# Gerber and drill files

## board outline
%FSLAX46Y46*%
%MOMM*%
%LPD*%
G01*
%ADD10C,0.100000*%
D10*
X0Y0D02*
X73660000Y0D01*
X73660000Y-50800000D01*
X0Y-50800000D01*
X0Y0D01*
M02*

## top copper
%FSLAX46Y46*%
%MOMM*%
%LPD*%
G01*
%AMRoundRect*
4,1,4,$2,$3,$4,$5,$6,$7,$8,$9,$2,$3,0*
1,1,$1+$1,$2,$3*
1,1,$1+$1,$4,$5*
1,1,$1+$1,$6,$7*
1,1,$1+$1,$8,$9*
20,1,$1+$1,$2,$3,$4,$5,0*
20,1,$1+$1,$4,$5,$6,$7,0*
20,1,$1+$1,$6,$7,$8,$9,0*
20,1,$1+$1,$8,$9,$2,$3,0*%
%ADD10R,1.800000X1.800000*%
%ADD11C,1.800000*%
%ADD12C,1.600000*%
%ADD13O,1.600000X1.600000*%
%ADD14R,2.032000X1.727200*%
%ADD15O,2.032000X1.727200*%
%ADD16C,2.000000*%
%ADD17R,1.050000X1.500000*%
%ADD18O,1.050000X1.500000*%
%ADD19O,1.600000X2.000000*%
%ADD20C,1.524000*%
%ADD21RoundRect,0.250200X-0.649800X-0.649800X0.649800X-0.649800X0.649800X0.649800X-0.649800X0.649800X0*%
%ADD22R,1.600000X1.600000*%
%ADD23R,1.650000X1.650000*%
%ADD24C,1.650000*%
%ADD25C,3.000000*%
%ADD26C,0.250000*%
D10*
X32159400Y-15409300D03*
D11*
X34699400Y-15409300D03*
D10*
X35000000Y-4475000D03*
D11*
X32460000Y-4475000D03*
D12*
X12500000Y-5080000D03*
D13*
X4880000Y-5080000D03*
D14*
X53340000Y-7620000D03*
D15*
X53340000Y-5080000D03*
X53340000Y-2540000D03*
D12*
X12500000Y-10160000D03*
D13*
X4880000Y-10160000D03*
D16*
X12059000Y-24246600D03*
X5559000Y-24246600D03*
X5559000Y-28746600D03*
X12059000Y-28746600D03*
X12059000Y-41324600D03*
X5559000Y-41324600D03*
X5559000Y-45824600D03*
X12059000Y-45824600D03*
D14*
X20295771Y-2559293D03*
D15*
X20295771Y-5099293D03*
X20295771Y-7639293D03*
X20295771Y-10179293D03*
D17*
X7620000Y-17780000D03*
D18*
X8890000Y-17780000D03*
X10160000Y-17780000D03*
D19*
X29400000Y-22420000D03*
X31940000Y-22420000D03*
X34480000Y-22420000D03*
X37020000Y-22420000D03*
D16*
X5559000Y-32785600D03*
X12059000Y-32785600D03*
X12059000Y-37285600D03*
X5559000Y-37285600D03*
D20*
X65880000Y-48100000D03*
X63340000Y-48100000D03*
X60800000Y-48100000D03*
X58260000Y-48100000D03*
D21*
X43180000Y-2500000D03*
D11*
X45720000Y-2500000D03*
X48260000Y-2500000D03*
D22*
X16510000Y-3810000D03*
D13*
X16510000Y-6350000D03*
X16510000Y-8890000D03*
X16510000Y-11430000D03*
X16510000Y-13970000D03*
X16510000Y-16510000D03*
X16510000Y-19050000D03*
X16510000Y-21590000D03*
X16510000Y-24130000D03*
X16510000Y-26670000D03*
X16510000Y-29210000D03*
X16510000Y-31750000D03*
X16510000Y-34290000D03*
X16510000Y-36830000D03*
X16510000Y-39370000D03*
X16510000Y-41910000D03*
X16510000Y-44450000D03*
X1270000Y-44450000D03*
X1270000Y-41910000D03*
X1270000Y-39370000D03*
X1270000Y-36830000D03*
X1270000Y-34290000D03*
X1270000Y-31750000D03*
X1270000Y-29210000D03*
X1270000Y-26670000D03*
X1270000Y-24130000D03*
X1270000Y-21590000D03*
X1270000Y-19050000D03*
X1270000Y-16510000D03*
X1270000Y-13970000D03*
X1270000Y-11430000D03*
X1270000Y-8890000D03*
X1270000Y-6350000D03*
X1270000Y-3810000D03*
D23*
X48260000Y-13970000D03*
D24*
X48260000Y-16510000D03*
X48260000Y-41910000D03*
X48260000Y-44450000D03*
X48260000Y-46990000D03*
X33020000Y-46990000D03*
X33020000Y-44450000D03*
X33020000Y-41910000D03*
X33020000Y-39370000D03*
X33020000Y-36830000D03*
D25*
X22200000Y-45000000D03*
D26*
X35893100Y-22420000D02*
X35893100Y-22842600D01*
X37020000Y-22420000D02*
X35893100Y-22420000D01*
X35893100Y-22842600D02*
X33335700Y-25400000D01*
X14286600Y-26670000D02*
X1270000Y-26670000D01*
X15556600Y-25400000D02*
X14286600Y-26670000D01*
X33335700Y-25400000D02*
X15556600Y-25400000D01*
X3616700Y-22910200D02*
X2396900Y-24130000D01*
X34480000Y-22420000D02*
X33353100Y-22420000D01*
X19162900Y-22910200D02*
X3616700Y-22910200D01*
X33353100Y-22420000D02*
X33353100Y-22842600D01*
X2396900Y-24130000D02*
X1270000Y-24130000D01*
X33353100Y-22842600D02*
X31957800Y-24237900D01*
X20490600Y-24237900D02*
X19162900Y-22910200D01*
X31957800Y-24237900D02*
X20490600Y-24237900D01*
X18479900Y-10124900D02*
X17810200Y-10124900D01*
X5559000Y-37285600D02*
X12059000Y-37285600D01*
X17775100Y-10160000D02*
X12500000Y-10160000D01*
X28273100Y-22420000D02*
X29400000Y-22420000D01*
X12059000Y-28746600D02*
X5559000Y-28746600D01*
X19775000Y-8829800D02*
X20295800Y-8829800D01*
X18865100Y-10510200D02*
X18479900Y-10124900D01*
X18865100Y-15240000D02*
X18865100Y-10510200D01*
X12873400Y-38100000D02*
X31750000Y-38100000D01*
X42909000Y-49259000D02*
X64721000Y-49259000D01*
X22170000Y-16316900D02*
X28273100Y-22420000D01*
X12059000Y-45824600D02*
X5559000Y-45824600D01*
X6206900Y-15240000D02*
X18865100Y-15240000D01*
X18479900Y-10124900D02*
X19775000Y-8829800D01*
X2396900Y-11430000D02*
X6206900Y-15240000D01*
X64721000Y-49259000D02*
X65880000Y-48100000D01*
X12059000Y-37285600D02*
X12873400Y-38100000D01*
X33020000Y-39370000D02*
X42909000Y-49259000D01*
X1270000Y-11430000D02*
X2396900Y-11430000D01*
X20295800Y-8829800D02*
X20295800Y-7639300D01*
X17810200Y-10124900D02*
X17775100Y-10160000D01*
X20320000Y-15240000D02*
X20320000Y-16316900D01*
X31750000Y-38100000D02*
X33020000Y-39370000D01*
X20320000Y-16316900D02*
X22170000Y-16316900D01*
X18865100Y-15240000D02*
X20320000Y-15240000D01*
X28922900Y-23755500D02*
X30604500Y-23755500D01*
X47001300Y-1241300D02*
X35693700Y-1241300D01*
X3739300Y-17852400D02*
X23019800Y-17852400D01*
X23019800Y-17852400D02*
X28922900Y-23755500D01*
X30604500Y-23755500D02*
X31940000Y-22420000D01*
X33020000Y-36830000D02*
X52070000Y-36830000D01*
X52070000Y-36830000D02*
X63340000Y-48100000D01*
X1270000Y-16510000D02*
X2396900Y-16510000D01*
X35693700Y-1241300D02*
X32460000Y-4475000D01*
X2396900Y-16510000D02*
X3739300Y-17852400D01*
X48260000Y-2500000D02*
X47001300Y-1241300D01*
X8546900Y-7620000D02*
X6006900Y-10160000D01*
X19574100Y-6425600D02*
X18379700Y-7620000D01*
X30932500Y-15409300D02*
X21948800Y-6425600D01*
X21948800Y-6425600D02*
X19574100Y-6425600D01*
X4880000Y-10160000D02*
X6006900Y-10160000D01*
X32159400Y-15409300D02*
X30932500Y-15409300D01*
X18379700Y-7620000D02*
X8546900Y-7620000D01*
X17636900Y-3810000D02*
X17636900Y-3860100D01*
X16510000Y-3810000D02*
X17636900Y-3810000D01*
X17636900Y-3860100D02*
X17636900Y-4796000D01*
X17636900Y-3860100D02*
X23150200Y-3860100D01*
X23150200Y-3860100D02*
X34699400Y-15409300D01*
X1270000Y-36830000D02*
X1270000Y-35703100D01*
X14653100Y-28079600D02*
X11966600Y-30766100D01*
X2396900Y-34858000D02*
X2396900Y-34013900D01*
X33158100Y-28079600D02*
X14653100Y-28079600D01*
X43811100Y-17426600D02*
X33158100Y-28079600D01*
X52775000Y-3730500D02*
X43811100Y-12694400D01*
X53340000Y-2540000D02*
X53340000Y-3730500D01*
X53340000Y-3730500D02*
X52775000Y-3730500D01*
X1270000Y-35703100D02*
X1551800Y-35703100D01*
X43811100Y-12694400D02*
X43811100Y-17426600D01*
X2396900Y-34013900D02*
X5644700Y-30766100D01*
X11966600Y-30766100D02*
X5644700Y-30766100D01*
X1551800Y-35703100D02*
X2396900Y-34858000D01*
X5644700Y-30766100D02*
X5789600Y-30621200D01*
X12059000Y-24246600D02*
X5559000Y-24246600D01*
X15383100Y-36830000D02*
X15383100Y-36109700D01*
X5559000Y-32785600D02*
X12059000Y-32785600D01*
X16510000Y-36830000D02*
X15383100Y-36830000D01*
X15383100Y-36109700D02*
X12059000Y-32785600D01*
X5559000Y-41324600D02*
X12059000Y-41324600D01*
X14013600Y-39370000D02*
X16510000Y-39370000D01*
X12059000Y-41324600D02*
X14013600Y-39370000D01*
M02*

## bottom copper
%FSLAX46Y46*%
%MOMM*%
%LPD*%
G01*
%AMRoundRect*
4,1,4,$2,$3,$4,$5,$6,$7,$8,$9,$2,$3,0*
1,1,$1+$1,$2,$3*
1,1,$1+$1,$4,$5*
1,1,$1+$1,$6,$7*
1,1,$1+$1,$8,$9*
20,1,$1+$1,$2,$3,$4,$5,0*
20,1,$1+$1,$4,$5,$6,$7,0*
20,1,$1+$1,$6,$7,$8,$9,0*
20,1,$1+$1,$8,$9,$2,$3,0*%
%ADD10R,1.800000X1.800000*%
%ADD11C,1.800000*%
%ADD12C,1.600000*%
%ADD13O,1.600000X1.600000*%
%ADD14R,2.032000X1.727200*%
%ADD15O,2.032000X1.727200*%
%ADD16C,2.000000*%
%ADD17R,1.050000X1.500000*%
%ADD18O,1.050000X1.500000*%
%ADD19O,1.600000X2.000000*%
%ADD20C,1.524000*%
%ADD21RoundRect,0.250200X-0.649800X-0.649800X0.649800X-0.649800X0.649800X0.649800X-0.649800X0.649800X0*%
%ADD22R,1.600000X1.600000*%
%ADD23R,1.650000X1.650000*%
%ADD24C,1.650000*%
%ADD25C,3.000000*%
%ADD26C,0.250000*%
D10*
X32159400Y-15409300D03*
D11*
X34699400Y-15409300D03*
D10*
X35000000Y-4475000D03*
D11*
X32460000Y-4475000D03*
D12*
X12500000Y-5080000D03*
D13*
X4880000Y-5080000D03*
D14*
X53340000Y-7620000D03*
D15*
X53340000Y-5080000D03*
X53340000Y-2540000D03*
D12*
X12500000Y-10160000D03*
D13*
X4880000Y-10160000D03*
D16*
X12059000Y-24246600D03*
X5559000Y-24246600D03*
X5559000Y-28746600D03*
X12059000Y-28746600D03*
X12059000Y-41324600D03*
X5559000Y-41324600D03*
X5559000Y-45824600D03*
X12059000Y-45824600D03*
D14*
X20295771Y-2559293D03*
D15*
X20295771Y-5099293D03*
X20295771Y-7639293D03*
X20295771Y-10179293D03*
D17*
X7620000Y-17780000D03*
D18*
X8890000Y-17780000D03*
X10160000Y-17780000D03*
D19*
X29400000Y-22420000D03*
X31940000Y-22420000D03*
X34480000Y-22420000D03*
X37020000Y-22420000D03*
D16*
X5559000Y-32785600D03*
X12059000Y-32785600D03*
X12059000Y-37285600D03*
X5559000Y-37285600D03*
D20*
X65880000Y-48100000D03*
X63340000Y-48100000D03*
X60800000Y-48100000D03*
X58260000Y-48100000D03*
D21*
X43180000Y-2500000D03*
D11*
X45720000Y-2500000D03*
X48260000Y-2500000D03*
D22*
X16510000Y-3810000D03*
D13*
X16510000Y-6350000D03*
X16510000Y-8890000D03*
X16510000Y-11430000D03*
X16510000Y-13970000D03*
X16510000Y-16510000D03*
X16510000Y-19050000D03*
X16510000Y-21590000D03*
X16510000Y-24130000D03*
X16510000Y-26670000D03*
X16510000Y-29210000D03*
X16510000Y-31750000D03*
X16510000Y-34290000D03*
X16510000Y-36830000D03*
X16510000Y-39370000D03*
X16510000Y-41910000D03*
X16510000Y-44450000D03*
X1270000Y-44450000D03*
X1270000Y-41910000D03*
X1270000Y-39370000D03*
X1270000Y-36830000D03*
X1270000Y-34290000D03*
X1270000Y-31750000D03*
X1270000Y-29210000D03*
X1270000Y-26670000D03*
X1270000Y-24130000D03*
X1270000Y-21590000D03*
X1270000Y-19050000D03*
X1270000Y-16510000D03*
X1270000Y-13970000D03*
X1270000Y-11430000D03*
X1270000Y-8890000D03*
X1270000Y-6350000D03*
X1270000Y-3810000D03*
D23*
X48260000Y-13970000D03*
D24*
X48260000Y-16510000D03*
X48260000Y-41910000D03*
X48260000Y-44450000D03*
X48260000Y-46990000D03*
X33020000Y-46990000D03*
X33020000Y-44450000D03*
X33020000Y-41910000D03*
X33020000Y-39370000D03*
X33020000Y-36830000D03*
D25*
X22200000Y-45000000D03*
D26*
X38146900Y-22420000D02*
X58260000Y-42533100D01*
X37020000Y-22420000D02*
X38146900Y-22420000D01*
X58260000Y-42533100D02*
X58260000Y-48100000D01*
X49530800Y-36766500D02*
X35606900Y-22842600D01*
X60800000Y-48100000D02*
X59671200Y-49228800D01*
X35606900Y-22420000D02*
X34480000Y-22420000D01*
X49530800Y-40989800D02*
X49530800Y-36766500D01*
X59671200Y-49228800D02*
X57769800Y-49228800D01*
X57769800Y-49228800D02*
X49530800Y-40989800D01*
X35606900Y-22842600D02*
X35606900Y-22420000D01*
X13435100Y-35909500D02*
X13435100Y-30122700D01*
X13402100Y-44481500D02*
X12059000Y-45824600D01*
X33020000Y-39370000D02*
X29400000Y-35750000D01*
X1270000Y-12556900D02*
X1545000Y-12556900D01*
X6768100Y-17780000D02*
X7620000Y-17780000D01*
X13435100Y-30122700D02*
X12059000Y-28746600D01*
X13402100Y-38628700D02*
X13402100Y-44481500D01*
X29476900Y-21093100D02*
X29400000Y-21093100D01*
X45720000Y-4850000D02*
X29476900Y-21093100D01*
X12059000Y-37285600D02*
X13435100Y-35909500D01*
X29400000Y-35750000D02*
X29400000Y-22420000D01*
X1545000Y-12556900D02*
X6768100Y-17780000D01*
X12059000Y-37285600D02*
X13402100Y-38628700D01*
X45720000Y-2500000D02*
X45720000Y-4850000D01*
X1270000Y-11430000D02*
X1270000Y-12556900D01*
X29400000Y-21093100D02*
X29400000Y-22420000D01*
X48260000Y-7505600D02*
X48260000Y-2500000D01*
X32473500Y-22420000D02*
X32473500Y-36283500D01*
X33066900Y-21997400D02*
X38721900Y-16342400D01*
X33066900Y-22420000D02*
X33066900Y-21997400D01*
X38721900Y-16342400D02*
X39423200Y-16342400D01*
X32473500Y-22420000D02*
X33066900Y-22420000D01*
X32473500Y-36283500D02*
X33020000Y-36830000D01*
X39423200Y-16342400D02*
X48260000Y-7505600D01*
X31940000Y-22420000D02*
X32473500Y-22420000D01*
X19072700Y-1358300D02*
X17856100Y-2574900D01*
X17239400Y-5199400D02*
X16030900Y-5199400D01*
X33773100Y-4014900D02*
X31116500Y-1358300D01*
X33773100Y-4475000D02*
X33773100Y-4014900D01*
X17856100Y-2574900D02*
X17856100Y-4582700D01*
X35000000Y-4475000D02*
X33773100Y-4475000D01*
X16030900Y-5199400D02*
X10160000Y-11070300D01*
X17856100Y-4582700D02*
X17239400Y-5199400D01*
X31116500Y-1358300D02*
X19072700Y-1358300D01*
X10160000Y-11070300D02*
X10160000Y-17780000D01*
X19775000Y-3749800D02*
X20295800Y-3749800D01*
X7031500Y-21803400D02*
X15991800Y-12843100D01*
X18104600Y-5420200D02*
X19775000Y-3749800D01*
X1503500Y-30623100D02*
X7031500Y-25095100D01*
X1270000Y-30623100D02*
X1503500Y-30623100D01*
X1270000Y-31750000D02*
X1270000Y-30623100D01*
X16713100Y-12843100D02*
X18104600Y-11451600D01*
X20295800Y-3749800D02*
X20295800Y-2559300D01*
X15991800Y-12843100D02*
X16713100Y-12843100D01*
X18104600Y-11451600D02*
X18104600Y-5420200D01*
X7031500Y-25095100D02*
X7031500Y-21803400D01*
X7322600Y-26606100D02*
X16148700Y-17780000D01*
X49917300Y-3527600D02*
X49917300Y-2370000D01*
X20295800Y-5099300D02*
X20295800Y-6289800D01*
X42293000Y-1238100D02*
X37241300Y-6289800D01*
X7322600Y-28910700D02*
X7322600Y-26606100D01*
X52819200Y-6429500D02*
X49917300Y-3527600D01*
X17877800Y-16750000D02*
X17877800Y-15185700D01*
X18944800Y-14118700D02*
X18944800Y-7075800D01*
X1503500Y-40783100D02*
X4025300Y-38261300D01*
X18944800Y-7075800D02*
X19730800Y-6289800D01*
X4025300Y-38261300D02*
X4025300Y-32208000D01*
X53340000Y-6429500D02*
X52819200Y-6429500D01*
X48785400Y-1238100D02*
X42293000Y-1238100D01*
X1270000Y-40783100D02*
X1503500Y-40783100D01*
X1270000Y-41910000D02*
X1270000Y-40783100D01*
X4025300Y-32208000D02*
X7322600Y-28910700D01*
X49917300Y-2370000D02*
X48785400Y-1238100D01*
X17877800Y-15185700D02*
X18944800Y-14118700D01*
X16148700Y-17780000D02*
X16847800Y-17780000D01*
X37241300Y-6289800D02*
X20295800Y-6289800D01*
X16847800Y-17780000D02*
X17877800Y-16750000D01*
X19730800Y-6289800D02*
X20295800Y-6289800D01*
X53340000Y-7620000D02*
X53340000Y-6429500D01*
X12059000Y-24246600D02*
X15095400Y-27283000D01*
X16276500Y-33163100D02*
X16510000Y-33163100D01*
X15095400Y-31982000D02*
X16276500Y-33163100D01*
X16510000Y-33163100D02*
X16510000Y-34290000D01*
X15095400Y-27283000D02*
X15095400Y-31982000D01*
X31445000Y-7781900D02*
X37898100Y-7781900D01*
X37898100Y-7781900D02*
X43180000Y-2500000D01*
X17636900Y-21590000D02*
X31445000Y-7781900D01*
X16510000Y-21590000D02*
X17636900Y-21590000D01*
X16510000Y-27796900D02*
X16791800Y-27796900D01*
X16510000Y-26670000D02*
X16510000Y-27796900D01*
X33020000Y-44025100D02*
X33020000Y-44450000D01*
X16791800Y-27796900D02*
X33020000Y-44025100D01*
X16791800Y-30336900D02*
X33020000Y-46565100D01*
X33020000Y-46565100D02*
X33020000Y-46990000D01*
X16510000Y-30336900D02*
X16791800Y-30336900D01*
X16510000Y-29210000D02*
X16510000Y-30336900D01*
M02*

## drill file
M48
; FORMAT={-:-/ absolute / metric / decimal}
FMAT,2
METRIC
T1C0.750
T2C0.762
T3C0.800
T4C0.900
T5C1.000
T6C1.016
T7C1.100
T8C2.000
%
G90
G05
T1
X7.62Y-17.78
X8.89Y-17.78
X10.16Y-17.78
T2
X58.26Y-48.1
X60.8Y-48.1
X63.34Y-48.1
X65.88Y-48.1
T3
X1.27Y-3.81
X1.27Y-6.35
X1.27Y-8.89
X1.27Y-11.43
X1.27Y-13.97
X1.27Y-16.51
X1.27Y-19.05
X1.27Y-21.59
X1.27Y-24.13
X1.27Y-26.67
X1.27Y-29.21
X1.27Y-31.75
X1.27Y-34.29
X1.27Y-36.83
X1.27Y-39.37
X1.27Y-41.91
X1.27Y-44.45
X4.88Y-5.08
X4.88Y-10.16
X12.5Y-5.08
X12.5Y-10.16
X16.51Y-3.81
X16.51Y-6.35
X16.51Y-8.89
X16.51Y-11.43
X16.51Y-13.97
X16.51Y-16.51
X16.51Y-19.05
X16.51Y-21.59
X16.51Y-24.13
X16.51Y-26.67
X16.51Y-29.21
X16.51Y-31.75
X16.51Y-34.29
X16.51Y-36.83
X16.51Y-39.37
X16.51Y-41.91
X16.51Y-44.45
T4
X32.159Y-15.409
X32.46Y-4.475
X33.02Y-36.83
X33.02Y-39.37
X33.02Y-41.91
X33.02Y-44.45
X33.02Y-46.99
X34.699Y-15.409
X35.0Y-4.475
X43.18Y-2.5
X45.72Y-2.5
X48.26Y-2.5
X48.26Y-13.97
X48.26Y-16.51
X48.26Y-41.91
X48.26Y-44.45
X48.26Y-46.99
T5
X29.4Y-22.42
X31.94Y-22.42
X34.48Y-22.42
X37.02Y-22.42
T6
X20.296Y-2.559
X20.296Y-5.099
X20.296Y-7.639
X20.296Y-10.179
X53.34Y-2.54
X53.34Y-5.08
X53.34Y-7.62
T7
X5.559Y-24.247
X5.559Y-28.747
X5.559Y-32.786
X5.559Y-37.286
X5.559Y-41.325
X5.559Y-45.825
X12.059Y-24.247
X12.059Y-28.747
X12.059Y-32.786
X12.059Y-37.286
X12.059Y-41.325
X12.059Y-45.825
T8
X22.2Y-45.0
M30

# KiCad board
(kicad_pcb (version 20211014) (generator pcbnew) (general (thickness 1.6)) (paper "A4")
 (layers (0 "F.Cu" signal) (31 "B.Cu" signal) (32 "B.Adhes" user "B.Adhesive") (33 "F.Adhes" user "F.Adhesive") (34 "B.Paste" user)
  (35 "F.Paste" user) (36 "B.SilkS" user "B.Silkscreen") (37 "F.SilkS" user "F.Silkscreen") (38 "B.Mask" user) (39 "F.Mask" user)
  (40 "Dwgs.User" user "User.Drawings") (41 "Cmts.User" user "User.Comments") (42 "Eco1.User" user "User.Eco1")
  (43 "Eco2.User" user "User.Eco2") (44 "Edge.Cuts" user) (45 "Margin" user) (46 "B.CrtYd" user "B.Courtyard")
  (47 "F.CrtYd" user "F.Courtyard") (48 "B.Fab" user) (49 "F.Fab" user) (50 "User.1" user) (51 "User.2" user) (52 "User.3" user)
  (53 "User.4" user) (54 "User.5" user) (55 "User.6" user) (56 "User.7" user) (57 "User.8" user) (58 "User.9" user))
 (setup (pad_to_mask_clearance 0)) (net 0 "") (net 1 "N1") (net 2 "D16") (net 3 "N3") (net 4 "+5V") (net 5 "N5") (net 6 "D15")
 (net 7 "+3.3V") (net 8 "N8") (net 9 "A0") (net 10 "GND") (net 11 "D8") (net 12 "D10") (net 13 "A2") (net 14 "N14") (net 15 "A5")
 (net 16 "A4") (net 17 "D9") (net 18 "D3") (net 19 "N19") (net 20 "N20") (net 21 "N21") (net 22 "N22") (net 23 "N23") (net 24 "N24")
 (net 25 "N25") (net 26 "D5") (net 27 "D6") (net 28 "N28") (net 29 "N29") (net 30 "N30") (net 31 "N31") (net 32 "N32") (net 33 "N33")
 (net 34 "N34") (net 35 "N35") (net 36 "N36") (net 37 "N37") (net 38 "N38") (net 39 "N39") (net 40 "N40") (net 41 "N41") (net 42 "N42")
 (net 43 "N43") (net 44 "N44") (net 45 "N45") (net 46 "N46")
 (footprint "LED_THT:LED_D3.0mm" (layer "F.Cu") (at 32.1594 15.4093)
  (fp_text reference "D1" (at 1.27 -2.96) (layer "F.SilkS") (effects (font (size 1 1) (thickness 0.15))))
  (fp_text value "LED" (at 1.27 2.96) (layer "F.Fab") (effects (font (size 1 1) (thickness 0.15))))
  (pad "1" thru_hole rect (at 0 0) (size 1.8 1.8) (drill 0.9) (layers *.Cu *.Mask) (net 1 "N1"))
  (pad "2" thru_hole circle (at 2.54 0) (size 1.8 1.8) (drill 0.9) (layers *.Cu *.Mask) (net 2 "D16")))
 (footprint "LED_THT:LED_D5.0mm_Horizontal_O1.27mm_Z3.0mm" (layer "F.Cu") (at 35 4.475 180)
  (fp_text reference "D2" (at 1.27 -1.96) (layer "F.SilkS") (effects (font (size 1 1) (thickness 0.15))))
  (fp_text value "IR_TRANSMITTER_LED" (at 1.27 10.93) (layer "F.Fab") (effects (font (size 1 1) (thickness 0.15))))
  (pad "1" thru_hole rect (at 0 0 180) (size 1.8 1.8) (drill 0.9) (layers *.Cu *.Mask) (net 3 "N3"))
  (pad "2" thru_hole circle (at 2.54 0 180) (size 1.8 1.8) (drill 0.9) (layers *.Cu *.Mask) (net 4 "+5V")))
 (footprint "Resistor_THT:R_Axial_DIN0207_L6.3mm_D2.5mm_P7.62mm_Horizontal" (layer "F.Cu") (at 12.5 5.08 180)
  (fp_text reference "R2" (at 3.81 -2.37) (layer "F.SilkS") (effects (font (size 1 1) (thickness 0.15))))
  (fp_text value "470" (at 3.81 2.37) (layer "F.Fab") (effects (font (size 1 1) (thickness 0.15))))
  (pad "1" thru_hole circle (at 0 0 180) (size 1.6 1.6) (drill 0.8) (layers *.Cu *.Mask) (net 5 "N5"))
  (pad "2" thru_hole oval (at 7.62 0 180) (size 1.6 1.6) (drill 0.8) (layers *.Cu *.Mask) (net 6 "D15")))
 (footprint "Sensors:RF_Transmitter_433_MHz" (layer "F.Cu") (at 53.34 5.08 90)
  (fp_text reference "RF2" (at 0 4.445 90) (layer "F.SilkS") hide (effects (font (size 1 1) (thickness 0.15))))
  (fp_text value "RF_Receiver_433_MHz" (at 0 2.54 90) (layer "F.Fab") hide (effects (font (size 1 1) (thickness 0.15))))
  (pad "1" thru_hole rect locked (at -2.54 0 180) (size 2.032 1.7272) (drill 1.016) (layers *.Cu *.Mask "F.SilkS") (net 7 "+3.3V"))
  (pad "2" thru_hole oval locked (at 0 0 180) (size 2.032 1.7272) (drill 1.016) (layers *.Cu *.Mask "F.SilkS") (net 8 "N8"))
  (pad "3" thru_hole oval locked (at 2.54 0 180) (size 2.032 1.7272) (drill 1.016) (layers *.Cu *.Mask "F.SilkS") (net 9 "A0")))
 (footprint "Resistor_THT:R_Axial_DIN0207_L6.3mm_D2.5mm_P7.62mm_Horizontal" (layer "F.Cu") (at 12.5 10.16 180)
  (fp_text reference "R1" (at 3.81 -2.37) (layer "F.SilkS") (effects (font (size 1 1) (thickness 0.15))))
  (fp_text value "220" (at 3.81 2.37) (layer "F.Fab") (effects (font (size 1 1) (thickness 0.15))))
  (pad "1" thru_hole circle (at 0 0 180) (size 1.6 1.6) (drill 0.8) (layers *.Cu *.Mask) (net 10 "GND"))
  (pad "2" thru_hole oval (at 7.62 0 180) (size 1.6 1.6) (drill 0.8) (layers *.Cu *.Mask) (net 1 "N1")))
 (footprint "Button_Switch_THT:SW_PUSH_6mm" (layer "F.Cu") (at 5.559 24.2466)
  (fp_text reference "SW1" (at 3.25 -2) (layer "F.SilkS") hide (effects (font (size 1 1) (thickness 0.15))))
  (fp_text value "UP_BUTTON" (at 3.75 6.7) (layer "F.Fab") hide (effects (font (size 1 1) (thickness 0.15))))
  (pad "1" thru_hole circle (at 6.5 0 90) (size 2 2) (drill 1.1) (layers *.Cu *.Mask) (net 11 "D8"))
  (pad "1" thru_hole circle (at 0 0 90) (size 2 2) (drill 1.1) (layers *.Cu *.Mask) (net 11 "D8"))
  (pad "2" thru_hole circle (at 0 4.5 90) (size 2 2) (drill 1.1) (layers *.Cu *.Mask) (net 10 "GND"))
  (pad "2" thru_hole circle (at 6.5 4.5 90) (size 2 2) (drill 1.1) (layers *.Cu *.Mask) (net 10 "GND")))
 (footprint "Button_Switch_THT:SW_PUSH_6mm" (layer "F.Cu") (at 5.559 41.3246)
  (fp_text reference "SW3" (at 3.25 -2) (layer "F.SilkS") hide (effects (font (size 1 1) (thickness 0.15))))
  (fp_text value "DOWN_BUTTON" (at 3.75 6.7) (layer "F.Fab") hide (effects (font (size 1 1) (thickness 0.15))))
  (pad "1" thru_hole circle (at 6.5 0 90) (size 2 2) (drill 1.1) (layers *.Cu *.Mask) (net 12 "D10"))
  (pad "1" thru_hole circle (at 0 0 90) (size 2 2) (drill 1.1) (layers *.Cu *.Mask) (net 12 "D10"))
  (pad "2" thru_hole circle (at 0 4.5 90) (size 2 2) (drill 1.1) (layers *.Cu *.Mask) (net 10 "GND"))
  (pad "2" thru_hole circle (at 6.5 4.5 90) (size 2 2) (drill 1.1) (layers *.Cu *.Mask) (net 10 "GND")))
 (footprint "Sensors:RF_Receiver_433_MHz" (layer "F.Cu") (at 20.32 7.62 -90)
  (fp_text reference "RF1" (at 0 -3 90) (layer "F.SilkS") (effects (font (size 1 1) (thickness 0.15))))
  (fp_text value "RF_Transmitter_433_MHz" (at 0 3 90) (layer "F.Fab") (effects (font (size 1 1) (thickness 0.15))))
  (pad "1" thru_hole rect locked (at -5.060707 0.024229) (size 2.032 1.7272) (drill 1.016) (layers *.Cu *.Mask "F.SilkS") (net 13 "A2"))
  (pad "2" thru_hole oval locked (at -2.520707 0.024229) (size 2.032 1.7272) (drill 1.016) (layers *.Cu *.Mask "F.SilkS") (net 7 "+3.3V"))
  (pad "3" thru_hole oval locked (at 0.019293 0.024229) (size 2.032 1.7272) (drill 1.016) (layers *.Cu *.Mask "F.SilkS") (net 10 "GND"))
  (pad "4" thru_hole oval locked (at 2.559293 0.024229) (size 2.032 1.7272) (drill 1.016) (layers *.Cu *.Mask "F.SilkS")))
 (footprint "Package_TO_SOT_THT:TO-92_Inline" (layer "F.Cu") (at 7.62 17.78)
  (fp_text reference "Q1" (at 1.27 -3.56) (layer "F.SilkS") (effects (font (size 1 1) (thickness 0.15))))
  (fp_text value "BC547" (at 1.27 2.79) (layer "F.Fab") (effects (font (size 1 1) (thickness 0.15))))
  (pad "1" thru_hole rect (at 0 0) (size 1.05 1.5) (drill 0.75) (layers *.Cu *.Mask) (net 10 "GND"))
  (pad "2" thru_hole oval (at 1.27 0) (size 1.05 1.5) (drill 0.75) (layers *.Cu *.Mask) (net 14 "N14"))
  (pad "3" thru_hole oval (at 2.54 0) (size 1.05 1.5) (drill 0.75) (layers *.Cu *.Mask) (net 3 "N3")))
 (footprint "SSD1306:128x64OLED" (layer "F.Cu") (at 33.02 33.02)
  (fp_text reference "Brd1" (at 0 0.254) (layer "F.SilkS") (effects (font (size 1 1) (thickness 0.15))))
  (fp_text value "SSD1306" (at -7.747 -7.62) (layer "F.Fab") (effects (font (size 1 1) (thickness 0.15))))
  (pad "1" thru_hole oval locked (at -3.62 -10.6 90) (size 2 1.6) (drill 1) (layers *.Cu *.Mask) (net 10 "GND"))
  (pad "2" thru_hole oval locked (at -1.08 -10.6 90) (size 2 1.6) (drill 1) (layers *.Cu *.Mask) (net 4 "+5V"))
  (pad "3" thru_hole oval locked (at 1.46 -10.6 90) (size 2 1.6) (drill 1) (layers *.Cu *.Mask) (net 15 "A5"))
  (pad "4" thru_hole oval locked (at 4 -10.6 90) (size 2 1.6) (drill 1) (layers *.Cu *.Mask) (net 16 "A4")))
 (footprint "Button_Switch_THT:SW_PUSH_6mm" (layer "F.Cu") (at 5.559 32.7856)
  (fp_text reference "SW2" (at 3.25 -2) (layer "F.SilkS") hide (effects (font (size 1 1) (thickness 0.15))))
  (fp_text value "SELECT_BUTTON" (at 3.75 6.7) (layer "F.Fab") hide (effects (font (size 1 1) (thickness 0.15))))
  (pad "1" thru_hole circle (at 0 0 90) (size 2 2) (drill 1.1) (layers *.Cu *.Mask) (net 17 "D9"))
  (pad "1" thru_hole circle (at 6.5 0 90) (size 2 2) (drill 1.1) (layers *.Cu *.Mask) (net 17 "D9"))
  (pad "2" thru_hole circle (at 6.5 4.5 90) (size 2 2) (drill 1.1) (layers *.Cu *.Mask) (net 10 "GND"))
  (pad "2" thru_hole circle (at 0 4.5 90) (size 2 2) (drill 1.1) (layers *.Cu *.Mask) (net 10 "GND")))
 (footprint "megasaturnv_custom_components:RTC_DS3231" (layer "F.Cu") (at 73.5 10 -90)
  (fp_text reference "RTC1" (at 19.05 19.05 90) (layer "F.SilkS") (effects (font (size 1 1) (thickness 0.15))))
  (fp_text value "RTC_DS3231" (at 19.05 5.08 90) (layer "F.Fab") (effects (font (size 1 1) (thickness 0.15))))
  (pad "1" thru_hole circle locked (at 38.1 7.62 270) (size 1.524 1.524) (drill 0.762) (layers *.Cu *.Mask) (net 10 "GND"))
  (pad "2" thru_hole circle locked (at 38.1 10.16 270) (size 1.524 1.524) (drill 0.762) (layers *.Cu *.Mask) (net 4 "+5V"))
  (pad "3" thru_hole circle locked (at 38.1 12.7 270) (size 1.524 1.524) (drill 0.762) (layers *.Cu *.Mask) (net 15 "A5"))
  (pad "4" thru_hole circle locked (at 38.1 15.24 270) (size 1.524 1.524) (drill 0.762) (layers *.Cu *.Mask) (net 16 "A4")))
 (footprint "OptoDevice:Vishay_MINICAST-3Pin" (layer "B.Cu") (at 43.18 2.5)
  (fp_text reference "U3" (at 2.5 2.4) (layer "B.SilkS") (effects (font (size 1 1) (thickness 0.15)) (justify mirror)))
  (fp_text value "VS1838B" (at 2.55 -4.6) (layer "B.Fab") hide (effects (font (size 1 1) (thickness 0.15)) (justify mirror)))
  (pad "1" thru_hole roundrect (at 0 0) (size 1.8 1.8) (drill 0.9) (layers *.Cu *.Mask) (roundrect_rratio 0.139) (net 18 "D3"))
  (pad "2" thru_hole circle (at 2.54 0) (size 1.8 1.8) (drill 0.9) (layers *.Cu *.Mask) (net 10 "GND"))
  (pad "3" thru_hole circle (at 5.08 0) (size 1.8 1.8) (drill 0.9) (layers *.Cu *.Mask) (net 4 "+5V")))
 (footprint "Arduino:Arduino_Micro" (layer "B.Cu") (at 16.51 3.81 180)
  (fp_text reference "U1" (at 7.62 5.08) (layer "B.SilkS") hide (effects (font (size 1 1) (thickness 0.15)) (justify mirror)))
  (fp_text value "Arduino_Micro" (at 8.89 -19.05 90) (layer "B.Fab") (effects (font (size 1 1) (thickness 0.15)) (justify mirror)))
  (pad "1" thru_hole rect locked (at 0 0 180) (size 1.6 1.6) (drill 0.8) (layers *.Cu *.Mask) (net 2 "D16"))
  (pad "2" thru_hole oval locked (at 0 -2.54 180) (size 1.6 1.6) (drill 0.8) (layers *.Cu *.Mask) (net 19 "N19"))
  (pad "3" thru_hole oval locked (at 0 -5.08 180) (size 1.6 1.6) (drill 0.8) (layers *.Cu *.Mask) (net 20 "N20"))
  (pad "4" thru_hole oval locked (at 0 -7.62 180) (size 1.6 1.6) (drill 0.8) (layers *.Cu *.Mask) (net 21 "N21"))
  (pad "5" thru_hole oval locked (at 0 -10.16 180) (size 1.6 1.6) (drill 0.8) (layers *.Cu *.Mask) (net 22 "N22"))
  (pad "6" thru_hole oval locked (at 0 -12.7 180) (size 1.6 1.6) (drill 0.8) (layers *.Cu *.Mask) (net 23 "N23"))
  (pad "7" thru_hole oval locked (at 0 -15.24 180) (size 1.6 1.6) (drill 0.8) (layers *.Cu *.Mask) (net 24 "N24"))
  (pad "8" thru_hole oval locked (at 0 -17.78 180) (size 1.6 1.6) (drill 0.8) (layers *.Cu *.Mask) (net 18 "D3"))
  (pad "9" thru_hole oval locked (at 0 -20.32 180) (size 1.6 1.6) (drill 0.8) (layers *.Cu *.Mask) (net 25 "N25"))
  (pad "10" thru_hole oval locked (at 0 -22.86 180) (size 1.6 1.6) (drill 0.8) (layers *.Cu *.Mask) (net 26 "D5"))
  (pad "11" thru_hole oval locked (at 0 -25.4 180) (size 1.6 1.6) (drill 0.8) (layers *.Cu *.Mask) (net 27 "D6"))
  (pad "12" thru_hole oval locked (at 0 -27.94 180) (size 1.6 1.6) (drill 0.8) (layers *.Cu *.Mask) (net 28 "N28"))
  (pad "13" thru_hole oval locked (at 0 -30.48 180) (size 1.6 1.6) (drill 0.8) (layers *.Cu *.Mask) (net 11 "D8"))
  (pad "14" thru_hole oval locked (at 0 -33.02 180) (size 1.6 1.6) (drill 0.8) (layers *.Cu *.Mask) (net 17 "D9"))
  (pad "15" thru_hole oval locked (at 0 -35.56 180) (size 1.6 1.6) (drill 0.8) (layers *.Cu *.Mask) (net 12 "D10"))
  (pad "16" thru_hole oval locked (at 0 -38.1 180) (size 1.6 1.6) (drill 0.8) (layers *.Cu *.Mask) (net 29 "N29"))
  (pad "17" thru_hole oval locked (at 0 -40.64 180) (size 1.6 1.6) (drill 0.8) (layers *.Cu *.Mask) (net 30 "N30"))
  (pad "18" thru_hole oval locked (at 15.24 -40.64 180) (size 1.6 1.6) (drill 0.8) (layers *.Cu *.Mask) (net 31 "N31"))
  (pad "19" thru_hole oval locked (at 15.24 -38.1 180) (size 1.6 1.6) (drill 0.8) (layers *.Cu *.Mask) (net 7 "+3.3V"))
  (pad "20" thru_hole oval locked (at 15.24 -35.56 180) (size 1.6 1.6) (drill 0.8) (layers *.Cu *.Mask) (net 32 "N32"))
  (pad "21" thru_hole oval locked (at 15.24 -33.02 180) (size 1.6 1.6) (drill 0.8) (layers *.Cu *.Mask) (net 9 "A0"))
  (pad "22" thru_hole oval locked (at 15.24 -30.48 180) (size 1.6 1.6) (drill 0.8) (layers *.Cu *.Mask) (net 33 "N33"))
  (pad "23" thru_hole oval locked (at 15.24 -27.94 180) (size 1.6 1.6) (drill 0.8) (layers *.Cu *.Mask) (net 13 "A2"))
  (pad "24" thru_hole oval locked (at 15.24 -25.4 180) (size 1.6 1.6) (drill 0.8) (layers *.Cu *.Mask) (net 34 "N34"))
  (pad "25" thru_hole oval locked (at 15.24 -22.86 180) (size 1.6 1.6) (drill 0.8) (layers *.Cu *.Mask) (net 16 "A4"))
  (pad "26" thru_hole oval locked (at 15.24 -20.32 180) (size 1.6 1.6) (drill 0.8) (layers *.Cu *.Mask) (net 15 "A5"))
  (pad "27" thru_hole oval locked (at 15.24 -17.78 180) (size 1.6 1.6) (drill 0.8) (layers *.Cu *.Mask) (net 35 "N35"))
  (pad "28" thru_hole oval locked (at 15.24 -15.24 180) (size 1.6 1.6) (drill 0.8) (layers *.Cu *.Mask) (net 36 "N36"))
  (pad "29" thru_hole oval locked (at 15.24 -12.7 180) (size 1.6 1.6) (drill 0.8) (layers *.Cu *.Mask) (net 4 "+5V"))
  (pad "30" thru_hole oval locked (at 15.24 -10.16 180) (size 1.6 1.6) (drill 0.8) (layers *.Cu *.Mask) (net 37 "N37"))
  (pad "31" thru_hole oval locked (at 15.24 -7.62 180) (size 1.6 1.6) (drill 0.8) (layers *.Cu *.Mask) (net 10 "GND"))
  (pad "32" thru_hole oval locked (at 15.24 -5.08 180) (size 1.6 1.6) (drill 0.8) (layers *.Cu *.Mask) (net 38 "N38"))
  (pad "33" thru_hole oval locked (at 15.24 -2.54 180) (size 1.6 1.6) (drill 0.8) (layers *.Cu *.Mask) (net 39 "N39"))
  (pad "34" thru_hole oval locked (at 15.24 0 180) (size 1.6 1.6) (drill 0.8) (layers *.Cu *.Mask) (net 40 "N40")))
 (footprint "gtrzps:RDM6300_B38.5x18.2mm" (layer "B.Cu") (at 48.26 13.97 -90)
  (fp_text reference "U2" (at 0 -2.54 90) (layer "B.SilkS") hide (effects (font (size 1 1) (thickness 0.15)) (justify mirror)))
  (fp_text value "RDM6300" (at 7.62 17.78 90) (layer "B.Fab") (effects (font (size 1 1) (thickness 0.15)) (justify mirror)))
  (pad "1" thru_hole rect locked (at 0 0 270) (size 1.65 1.65) (drill 0.9) (layers *.Cu *.Mask) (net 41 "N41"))
  (pad "2" thru_hole circle locked (at 2.54 0 270) (size 1.65 1.65) (drill 0.9) (layers *.Cu *.Mask) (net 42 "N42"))
  (pad "3" thru_hole circle locked (at 27.94 0 270) (size 1.65 1.65) (drill 0.9) (layers *.Cu *.Mask) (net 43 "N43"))
  (pad "4" thru_hole circle locked (at 30.48 0 270) (size 1.65 1.65) (drill 0.9) (layers *.Cu *.Mask) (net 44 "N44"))
  (pad "5" thru_hole circle locked (at 33.02 0 270) (size 1.65 1.65) (drill 0.9) (layers *.Cu *.Mask) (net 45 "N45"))
  (pad "6" thru_hole circle locked (at 33.02 15.24 270) (size 1.65 1.65) (drill 0.9) (layers *.Cu *.Mask) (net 27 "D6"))
  (pad "7" thru_hole circle locked (at 30.48 15.24 270) (size 1.65 1.65) (drill 0.9) (layers *.Cu *.Mask) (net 26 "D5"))
  (pad "8" thru_hole circle locked (at 27.94 15.24 270) (size 1.65 1.65) (drill 0.9) (layers *.Cu *.Mask) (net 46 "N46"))
  (pad "9" thru_hole circle locked (at 25.4 15.24 270) (size 1.65 1.65) (drill 0.9) (layers *.Cu *.Mask) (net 10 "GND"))
  (pad "10" thru_hole circle locked (at 22.86 15.24 270) (size 1.65 1.65) (drill 0.9) (layers *.Cu *.Mask) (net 4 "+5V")))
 (gr_rect (start 0 0) (end 73.66 50.8) (layer "Edge.Cuts") (width 0.1) (fill none))
 (via (at 22.2 45) (size 3) (drill 2) (layers "F.Cu" "B.Cu") (free) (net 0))
 (segment (start 35.8931 22.42) (end 35.8931 22.8426) (width 0.25) (layer "F.Cu") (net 16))
 (segment (start 37.02 22.42) (end 35.8931 22.42) (width 0.25) (layer "F.Cu") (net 16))
 (segment (start 35.8931 22.8426) (end 33.3357 25.4) (width 0.25) (layer "F.Cu") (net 16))
 (segment (start 14.2866 26.67) (end 1.27 26.67) (width 0.25) (layer "F.Cu") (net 16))
 (segment (start 15.5566 25.4) (end 14.2866 26.67) (width 0.25) (layer "F.Cu") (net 16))
 (segment (start 33.3357 25.4) (end 15.5566 25.4) (width 0.25) (layer "F.Cu") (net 16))
 (segment (start 38.1469 22.42) (end 58.26 42.5331) (width 0.25) (layer "B.Cu") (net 16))
 (segment (start 37.02 22.42) (end 38.1469 22.42) (width 0.25) (layer "B.Cu") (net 16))
 (segment (start 58.26 42.5331) (end 58.26 48.1) (width 0.25) (layer "B.Cu") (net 16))
 (segment (start 3.6167 22.9102) (end 2.3969 24.13) (width 0.25) (layer "F.Cu") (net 15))
 (segment (start 34.48 22.42) (end 33.3531 22.42) (width 0.25) (layer "F.Cu") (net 15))
 (segment (start 19.1629 22.9102) (end 3.6167 22.9102) (width 0.25) (layer "F.Cu") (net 15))
 (segment (start 33.3531 22.42) (end 33.3531 22.8426) (width 0.25) (layer "F.Cu") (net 15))
 (segment (start 2.3969 24.13) (end 1.27 24.13) (width 0.25) (layer "F.Cu") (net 15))
 (segment (start 33.3531 22.8426) (end 31.9578 24.2379) (width 0.25) (layer "F.Cu") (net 15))
 (segment (start 20.4906 24.2379) (end 19.1629 22.9102) (width 0.25) (layer "F.Cu") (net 15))
 (segment (start 31.9578 24.2379) (end 20.4906 24.2379) (width 0.25) (layer "F.Cu") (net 15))
 (segment (start 49.5308 36.7665) (end 35.6069 22.8426) (width 0.25) (layer "B.Cu") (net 15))
 (segment (start 60.8 48.1) (end 59.6712 49.2288) (width 0.25) (layer "B.Cu") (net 15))
 (segment (start 35.6069 22.42) (end 34.48 22.42) (width 0.25) (layer "B.Cu") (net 15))
 (segment (start 49.5308 40.9898) (end 49.5308 36.7665) (width 0.25) (layer "B.Cu") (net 15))
 (segment (start 59.6712 49.2288) (end 57.7698 49.2288) (width 0.25) (layer "B.Cu") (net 15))
 (segment (start 57.7698 49.2288) (end 49.5308 40.9898) (width 0.25) (layer "B.Cu") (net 15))
 (segment (start 35.6069 22.8426) (end 35.6069 22.42) (width 0.25) (layer "B.Cu") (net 15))
 (segment (start 18.4799 10.1249) (end 17.8102 10.1249) (width 0.25) (layer "F.Cu") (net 10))
 (segment (start 5.559 37.2856) (end 12.059 37.2856) (width 0.25) (layer "F.Cu") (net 10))
 (segment (start 17.7751 10.16) (end 12.5 10.16) (width 0.25) (layer "F.Cu") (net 10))
 (segment (start 28.2731 22.42) (end 29.4 22.42) (width 0.25) (layer "F.Cu") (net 10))
 (segment (start 12.059 28.7466) (end 5.559 28.7466) (width 0.25) (layer "F.Cu") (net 10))
 (segment (start 19.775 8.8298) (end 20.2958 8.8298) (width 0.25) (layer "F.Cu") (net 10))
 (segment (start 18.8651 10.5102) (end 18.4799 10.1249) (width 0.25) (layer "F.Cu") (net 10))
 (segment (start 18.8651 15.24) (end 18.8651 10.5102) (width 0.25) (layer "F.Cu") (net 10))
 (segment (start 12.8734 38.1) (end 31.75 38.1) (width 0.25) (layer "F.Cu") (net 10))
 (segment (start 42.909 49.259) (end 64.721 49.259) (width 0.25) (layer "F.Cu") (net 10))
 (segment (start 22.17 16.3169) (end 28.2731 22.42) (width 0.25) (layer "F.Cu") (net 10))
 (segment (start 12.059 45.8246) (end 5.559 45.8246) (width 0.25) (layer "F.Cu") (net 10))
 (segment (start 6.2069 15.24) (end 18.8651 15.24) (width 0.25) (layer "F.Cu") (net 10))
 (segment (start 18.4799 10.1249) (end 19.775 8.8298) (width 0.25) (layer "F.Cu") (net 10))
 (segment (start 2.3969 11.43) (end 6.2069 15.24) (width 0.25) (layer "F.Cu") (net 10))
 (segment (start 64.721 49.259) (end 65.88 48.1) (width 0.25) (layer "F.Cu") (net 10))
 (segment (start 12.059 37.2856) (end 12.8734 38.1) (width 0.25) (layer "F.Cu") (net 10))
 (segment (start 33.02 39.37) (end 42.909 49.259) (width 0.25) (layer "F.Cu") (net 10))
 (segment (start 1.27 11.43) (end 2.3969 11.43) (width 0.25) (layer "F.Cu") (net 10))
 (segment (start 20.2958 8.8298) (end 20.2958 7.6393) (width 0.25) (layer "F.Cu") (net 10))
 (segment (start 17.8102 10.1249) (end 17.7751 10.16) (width 0.25) (layer "F.Cu") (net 10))
 (segment (start 20.32 15.24) (end 20.32 16.3169) (width 0.25) (layer "F.Cu") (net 10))
 (segment (start 31.75 38.1) (end 33.02 39.37) (width 0.25) (layer "F.Cu") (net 10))
 (segment (start 20.32 16.3169) (end 22.17 16.3169) (width 0.25) (layer "F.Cu") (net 10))
 (segment (start 18.8651 15.24) (end 20.32 15.24) (width 0.25) (layer "F.Cu") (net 10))
 (segment (start 13.4351 35.9095) (end 13.4351 30.1227) (width 0.25) (layer "B.Cu") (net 10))
 (segment (start 13.4021 44.4815) (end 12.059 45.8246) (width 0.25) (layer "B.Cu") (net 10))
 (segment (start 33.02 39.37) (end 29.4 35.75) (width 0.25) (layer "B.Cu") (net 10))
 (segment (start 1.27 12.5569) (end 1.545 12.5569) (width 0.25) (layer "B.Cu") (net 10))
 (segment (start 6.7681 17.78) (end 7.62 17.78) (width 0.25) (layer "B.Cu") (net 10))
 (segment (start 13.4351 30.1227) (end 12.059 28.7466) (width 0.25) (layer "B.Cu") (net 10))
 (segment (start 13.4021 38.6287) (end 13.4021 44.4815) (width 0.25) (layer "B.Cu") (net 10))
 (segment (start 29.4769 21.0931) (end 29.4 21.0931) (width 0.25) (layer "B.Cu") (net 10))
 (segment (start 45.72 4.85) (end 29.4769 21.0931) (width 0.25) (layer "B.Cu") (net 10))
 (segment (start 12.059 37.2856) (end 13.4351 35.9095) (width 0.25) (layer "B.Cu") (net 10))
 (segment (start 29.4 35.75) (end 29.4 22.42) (width 0.25) (layer "B.Cu") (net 10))
 (segment (start 1.545 12.5569) (end 6.7681 17.78) (width 0.25) (layer "B.Cu") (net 10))
 (segment (start 12.059 37.2856) (end 13.4021 38.6287) (width 0.25) (layer "B.Cu") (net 10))
 (segment (start 45.72 2.5) (end 45.72 4.85) (width 0.25) (layer "B.Cu") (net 10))
 (segment (start 1.27 11.43) (end 1.27 12.5569) (width 0.25) (layer "B.Cu") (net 10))
 (segment (start 29.4 21.0931) (end 29.4 22.42) (width 0.25) (layer "B.Cu") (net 10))
 (segment (start 28.9229 23.7555) (end 30.6045 23.7555) (width 0.25) (layer "F.Cu") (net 4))
 (segment (start 47.0013 1.2413) (end 35.6937 1.2413) (width 0.25) (layer "F.Cu") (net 4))
 (segment (start 3.7393 17.8524) (end 23.0198 17.8524) (width 0.25) (layer "F.Cu") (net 4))
 (segment (start 23.0198 17.8524) (end 28.9229 23.7555) (width 0.25) (layer "F.Cu") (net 4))
 (segment (start 30.6045 23.7555) (end 31.94 22.42) (width 0.25) (layer "F.Cu") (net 4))
 (segment (start 33.02 36.83) (end 52.07 36.83) (width 0.25) (layer "F.Cu") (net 4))
 (segment (start 52.07 36.83) (end 63.34 48.1) (width 0.25) (layer "F.Cu") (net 4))
 (segment (start 1.27 16.51) (end 2.3969 16.51) (width 0.25) (layer "F.Cu") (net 4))
 (segment (start 35.6937 1.2413) (end 32.46 4.475) (width 0.25) (layer "F.Cu") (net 4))
 (segment (start 2.3969 16.51) (end 3.7393 17.8524) (width 0.25) (layer "F.Cu") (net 4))
 (segment (start 48.26 2.5) (end 47.0013 1.2413) (width 0.25) (layer "F.Cu") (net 4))
 (segment (start 48.26 7.5056) (end 48.26 2.5) (width 0.25) (layer "B.Cu") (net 4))
 (segment (start 32.4735 22.42) (end 32.4735 36.2835) (width 0.25) (layer "B.Cu") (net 4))
 (segment (start 33.0669 21.9974) (end 38.7219 16.3424) (width 0.25) (layer "B.Cu") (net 4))
 (segment (start 33.0669 22.42) (end 33.0669 21.9974) (width 0.25) (layer "B.Cu") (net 4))
 (segment (start 38.7219 16.3424) (end 39.4232 16.3424) (width 0.25) (layer "B.Cu") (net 4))
 (segment (start 32.4735 22.42) (end 33.0669 22.42) (width 0.25) (layer "B.Cu") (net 4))
 (segment (start 32.4735 36.2835) (end 33.02 36.83) (width 0.25) (layer "B.Cu") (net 4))
 (segment (start 39.4232 16.3424) (end 48.26 7.5056) (width 0.25) (layer "B.Cu") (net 4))
 (segment (start 31.94 22.42) (end 32.4735 22.42) (width 0.25) (layer "B.Cu") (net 4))
 (segment (start 8.5469 7.62) (end 6.0069 10.16) (width 0.25) (layer "F.Cu") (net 1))
 (segment (start 19.5741 6.4256) (end 18.3797 7.62) (width 0.25) (layer "F.Cu") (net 1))
 (segment (start 30.9325 15.4093) (end 21.9488 6.4256) (width 0.25) (layer "F.Cu") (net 1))
 (segment (start 21.9488 6.4256) (end 19.5741 6.4256) (width 0.25) (layer "F.Cu") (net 1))
 (segment (start 4.88 10.16) (end 6.0069 10.16) (width 0.25) (layer "F.Cu") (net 1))
 (segment (start 32.1594 15.4093) (end 30.9325 15.4093) (width 0.25) (layer "F.Cu") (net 1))
 (segment (start 18.3797 7.62) (end 8.5469 7.62) (width 0.25) (layer "F.Cu") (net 1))
 (segment (start 17.6369 3.81) (end 17.6369 3.8601) (width 0.25) (layer "F.Cu") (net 2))
 (segment (start 16.51 3.81) (end 17.6369 3.81) (width 0.25) (layer "F.Cu") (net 2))
 (segment (start 17.6369 3.8601) (end 17.6369 4.796) (width 0.25) (layer "F.Cu") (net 2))
 (segment (start 17.6369 3.8601) (end 23.1502 3.8601) (width 0.25) (layer "F.Cu") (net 2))
 (segment (start 23.1502 3.8601) (end 34.6994 15.4093) (width 0.25) (layer "F.Cu") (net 2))
 (segment (start 19.0727 1.3583) (end 17.8561 2.5749) (width 0.25) (layer "B.Cu") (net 3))
 (segment (start 17.2394 5.1994) (end 16.0309 5.1994) (width 0.25) (layer "B.Cu") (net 3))
 (segment (start 33.7731 4.0149) (end 31.1165 1.3583) (width 0.25) (layer "B.Cu") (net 3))
 (segment (start 33.7731 4.475) (end 33.7731 4.0149) (width 0.25) (layer "B.Cu") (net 3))
 (segment (start 17.8561 2.5749) (end 17.8561 4.5827) (width 0.25) (layer "B.Cu") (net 3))
 (segment (start 35 4.475) (end 33.7731 4.475) (width 0.25) (layer "B.Cu") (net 3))
 (segment (start 16.0309 5.1994) (end 10.16 11.0703) (width 0.25) (layer "B.Cu") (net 3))
 (segment (start 17.8561 4.5827) (end 17.2394 5.1994) (width 0.25) (layer "B.Cu") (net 3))
 (segment (start 31.1165 1.3583) (end 19.0727 1.3583) (width 0.25) (layer "B.Cu") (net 3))
 (segment (start 10.16 11.0703) (end 10.16 17.78) (width 0.25) (layer "B.Cu") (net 3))
 (segment (start 19.775 3.7498) (end 20.2958 3.7498) (width 0.25) (layer "B.Cu") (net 13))
 (segment (start 7.0315 21.8034) (end 15.9918 12.8431) (width 0.25) (layer "B.Cu") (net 13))
 (segment (start 18.1046 5.4202) (end 19.775 3.7498) (width 0.25) (layer "B.Cu") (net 13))
 (segment (start 1.5035 30.6231) (end 7.0315 25.0951) (width 0.25) (layer "B.Cu") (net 13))
 (segment (start 1.27 30.6231) (end 1.5035 30.6231) (width 0.25) (layer "B.Cu") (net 13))
 (segment (start 1.27 31.75) (end 1.27 30.6231) (width 0.25) (layer "B.Cu") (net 13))
 (segment (start 16.7131 12.8431) (end 18.1046 11.4516) (width 0.25) (layer "B.Cu") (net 13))
 (segment (start 20.2958 3.7498) (end 20.2958 2.5593) (width 0.25) (layer "B.Cu") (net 13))
 (segment (start 15.9918 12.8431) (end 16.7131 12.8431) (width 0.25) (layer "B.Cu") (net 13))
 (segment (start 18.1046 11.4516) (end 18.1046 5.4202) (width 0.25) (layer "B.Cu") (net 13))
 (segment (start 7.0315 25.0951) (end 7.0315 21.8034) (width 0.25) (layer "B.Cu") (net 13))
 (segment (start 7.3226 26.6061) (end 16.1487 17.78) (width 0.25) (layer "B.Cu") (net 7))
 (segment (start 49.9173 3.5276) (end 49.9173 2.37) (width 0.25) (layer "B.Cu") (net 7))
 (segment (start 20.2958 5.0993) (end 20.2958 6.2898) (width 0.25) (layer "B.Cu") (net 7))
 (segment (start 42.293 1.2381) (end 37.2413 6.2898) (width 0.25) (layer "B.Cu") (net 7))
 (segment (start 7.3226 28.9107) (end 7.3226 26.6061) (width 0.25) (layer "B.Cu") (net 7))
 (segment (start 52.8192 6.4295) (end 49.9173 3.5276) (width 0.25) (layer "B.Cu") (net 7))
 (segment (start 17.8778 16.75) (end 17.8778 15.1857) (width 0.25) (layer "B.Cu") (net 7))
 (segment (start 18.9448 14.1187) (end 18.9448 7.0758) (width 0.25) (layer "B.Cu") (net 7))
 (segment (start 1.5035 40.7831) (end 4.0253 38.2613) (width 0.25) (layer "B.Cu") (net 7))
 (segment (start 18.9448 7.0758) (end 19.7308 6.2898) (width 0.25) (layer "B.Cu") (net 7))
 (segment (start 4.0253 38.2613) (end 4.0253 32.208) (width 0.25) (layer "B.Cu") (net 7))
 (segment (start 53.34 6.4295) (end 52.8192 6.4295) (width 0.25) (layer "B.Cu") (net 7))
 (segment (start 48.7854 1.2381) (end 42.293 1.2381) (width 0.25) (layer "B.Cu") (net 7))
 (segment (start 1.27 40.7831) (end 1.5035 40.7831) (width 0.25) (layer "B.Cu") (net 7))
 (segment (start 1.27 41.91) (end 1.27 40.7831) (width 0.25) (layer "B.Cu") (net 7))
 (segment (start 4.0253 32.208) (end 7.3226 28.9107) (width 0.25) (layer "B.Cu") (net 7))
 (segment (start 49.9173 2.37) (end 48.7854 1.2381) (width 0.25) (layer "B.Cu") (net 7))
 (segment (start 17.8778 15.1857) (end 18.9448 14.1187) (width 0.25) (layer "B.Cu") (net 7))
 (segment (start 16.1487 17.78) (end 16.8478 17.78) (width 0.25) (layer "B.Cu") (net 7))
 (segment (start 37.2413 6.2898) (end 20.2958 6.2898) (width 0.25) (layer "B.Cu") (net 7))
 (segment (start 16.8478 17.78) (end 17.8778 16.75) (width 0.25) (layer "B.Cu") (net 7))
 (segment (start 19.7308 6.2898) (end 20.2958 6.2898) (width 0.25) (layer "B.Cu") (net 7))
 (segment (start 53.34 7.62) (end 53.34 6.4295) (width 0.25) (layer "B.Cu") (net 7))
 (segment (start 1.27 36.83) (end 1.27 35.7031) (width 0.25) (layer "F.Cu") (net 9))
 (segment (start 14.6531 28.0796) (end 11.9666 30.7661) (width 0.25) (layer "F.Cu") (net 9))
 (segment (start 2.3969 34.858) (end 2.3969 34.0139) (width 0.25) (layer "F.Cu") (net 9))
 (segment (start 33.1581 28.0796) (end 14.6531 28.0796) (width 0.25) (layer "F.Cu") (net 9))
 (segment (start 43.8111 17.4266) (end 33.1581 28.0796) (width 0.25) (layer "F.Cu") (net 9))
 (segment (start 52.775 3.7305) (end 43.8111 12.6944) (width 0.25) (layer "F.Cu") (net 9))
 (segment (start 53.34 2.54) (end 53.34 3.7305) (width 0.25) (layer "F.Cu") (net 9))
 (segment (start 53.34 3.7305) (end 52.775 3.7305) (width 0.25) (layer "F.Cu") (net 9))
 (segment (start 1.27 35.7031) (end 1.5518 35.7031) (width 0.25) (layer "F.Cu") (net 9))
 (segment (start 43.8111 12.6944) (end 43.8111 17.4266) (width 0.25) (layer "F.Cu") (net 9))
 (segment (start 2.3969 34.0139) (end 5.6447 30.7661) (width 0.25) (layer "F.Cu") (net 9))
 (segment (start 11.9666 30.7661) (end 5.6447 30.7661) (width 0.25) (layer "F.Cu") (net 9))
 (segment (start 1.5518 35.7031) (end 2.3969 34.858) (width 0.25) (layer "F.Cu") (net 9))
 (segment (start 5.6447 30.7661) (end 5.7896 30.6212) (width 0.25) (layer "F.Cu") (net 9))
 (segment (start 12.059 24.2466) (end 5.559 24.2466) (width 0.25) (layer "F.Cu") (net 11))
 (segment (start 12.059 24.2466) (end 15.0954 27.283) (width 0.25) (layer "B.Cu") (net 11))
 (segment (start 16.2765 33.1631) (end 16.51 33.1631) (width 0.25) (layer "B.Cu") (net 11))
 (segment (start 15.0954 31.982) (end 16.2765 33.1631) (width 0.25) (layer "B.Cu") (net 11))
 (segment (start 16.51 33.1631) (end 16.51 34.29) (width 0.25) (layer "B.Cu") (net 11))
 (segment (start 15.0954 27.283) (end 15.0954 31.982) (width 0.25) (layer "B.Cu") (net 11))
 (segment (start 15.3831 36.83) (end 15.3831 36.1097) (width 0.25) (layer "F.Cu") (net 17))
 (segment (start 5.559 32.7856) (end 12.059 32.7856) (width 0.25) (layer "F.Cu") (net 17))
 (segment (start 16.51 36.83) (end 15.3831 36.83) (width 0.25) (layer "F.Cu") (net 17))
 (segment (start 15.3831 36.1097) (end 12.059 32.7856) (width 0.25) (layer "F.Cu") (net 17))
 (segment (start 5.559 41.3246) (end 12.059 41.3246) (width 0.25) (layer "F.Cu") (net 12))
 (segment (start 14.0136 39.37) (end 16.51 39.37) (width 0.25) (layer "F.Cu") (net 12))
 (segment (start 12.059 41.3246) (end 14.0136 39.37) (width 0.25) (layer "F.Cu") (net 12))
 (segment (start 31.445 7.7819) (end 37.8981 7.7819) (width 0.25) (layer "B.Cu") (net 18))
 (segment (start 37.8981 7.7819) (end 43.18 2.5) (width 0.25) (layer "B.Cu") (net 18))
 (segment (start 17.6369 21.59) (end 31.445 7.7819) (width 0.25) (layer "B.Cu") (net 18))
 (segment (start 16.51 21.59) (end 17.6369 21.59) (width 0.25) (layer "B.Cu") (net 18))
 (segment (start 16.51 27.7969) (end 16.7918 27.7969) (width 0.25) (layer "B.Cu") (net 26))
 (segment (start 16.51 26.67) (end 16.51 27.7969) (width 0.25) (layer "B.Cu") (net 26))
 (segment (start 33.02 44.0251) (end 33.02 44.45) (width 0.25) (layer "B.Cu") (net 26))
 (segment (start 16.7918 27.7969) (end 33.02 44.0251) (width 0.25) (layer "B.Cu") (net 26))
 (segment (start 16.7918 30.3369) (end 33.02 46.5651) (width 0.25) (layer "B.Cu") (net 27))
 (segment (start 33.02 46.5651) (end 33.02 46.99) (width 0.25) (layer "B.Cu") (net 27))
 (segment (start 16.51 30.3369) (end 16.7918 30.3369) (width 0.25) (layer "B.Cu") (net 27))
 (segment (start 16.51 29.21) (end 16.51 30.3369) (width 0.25) (layer "B.Cu") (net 27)))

